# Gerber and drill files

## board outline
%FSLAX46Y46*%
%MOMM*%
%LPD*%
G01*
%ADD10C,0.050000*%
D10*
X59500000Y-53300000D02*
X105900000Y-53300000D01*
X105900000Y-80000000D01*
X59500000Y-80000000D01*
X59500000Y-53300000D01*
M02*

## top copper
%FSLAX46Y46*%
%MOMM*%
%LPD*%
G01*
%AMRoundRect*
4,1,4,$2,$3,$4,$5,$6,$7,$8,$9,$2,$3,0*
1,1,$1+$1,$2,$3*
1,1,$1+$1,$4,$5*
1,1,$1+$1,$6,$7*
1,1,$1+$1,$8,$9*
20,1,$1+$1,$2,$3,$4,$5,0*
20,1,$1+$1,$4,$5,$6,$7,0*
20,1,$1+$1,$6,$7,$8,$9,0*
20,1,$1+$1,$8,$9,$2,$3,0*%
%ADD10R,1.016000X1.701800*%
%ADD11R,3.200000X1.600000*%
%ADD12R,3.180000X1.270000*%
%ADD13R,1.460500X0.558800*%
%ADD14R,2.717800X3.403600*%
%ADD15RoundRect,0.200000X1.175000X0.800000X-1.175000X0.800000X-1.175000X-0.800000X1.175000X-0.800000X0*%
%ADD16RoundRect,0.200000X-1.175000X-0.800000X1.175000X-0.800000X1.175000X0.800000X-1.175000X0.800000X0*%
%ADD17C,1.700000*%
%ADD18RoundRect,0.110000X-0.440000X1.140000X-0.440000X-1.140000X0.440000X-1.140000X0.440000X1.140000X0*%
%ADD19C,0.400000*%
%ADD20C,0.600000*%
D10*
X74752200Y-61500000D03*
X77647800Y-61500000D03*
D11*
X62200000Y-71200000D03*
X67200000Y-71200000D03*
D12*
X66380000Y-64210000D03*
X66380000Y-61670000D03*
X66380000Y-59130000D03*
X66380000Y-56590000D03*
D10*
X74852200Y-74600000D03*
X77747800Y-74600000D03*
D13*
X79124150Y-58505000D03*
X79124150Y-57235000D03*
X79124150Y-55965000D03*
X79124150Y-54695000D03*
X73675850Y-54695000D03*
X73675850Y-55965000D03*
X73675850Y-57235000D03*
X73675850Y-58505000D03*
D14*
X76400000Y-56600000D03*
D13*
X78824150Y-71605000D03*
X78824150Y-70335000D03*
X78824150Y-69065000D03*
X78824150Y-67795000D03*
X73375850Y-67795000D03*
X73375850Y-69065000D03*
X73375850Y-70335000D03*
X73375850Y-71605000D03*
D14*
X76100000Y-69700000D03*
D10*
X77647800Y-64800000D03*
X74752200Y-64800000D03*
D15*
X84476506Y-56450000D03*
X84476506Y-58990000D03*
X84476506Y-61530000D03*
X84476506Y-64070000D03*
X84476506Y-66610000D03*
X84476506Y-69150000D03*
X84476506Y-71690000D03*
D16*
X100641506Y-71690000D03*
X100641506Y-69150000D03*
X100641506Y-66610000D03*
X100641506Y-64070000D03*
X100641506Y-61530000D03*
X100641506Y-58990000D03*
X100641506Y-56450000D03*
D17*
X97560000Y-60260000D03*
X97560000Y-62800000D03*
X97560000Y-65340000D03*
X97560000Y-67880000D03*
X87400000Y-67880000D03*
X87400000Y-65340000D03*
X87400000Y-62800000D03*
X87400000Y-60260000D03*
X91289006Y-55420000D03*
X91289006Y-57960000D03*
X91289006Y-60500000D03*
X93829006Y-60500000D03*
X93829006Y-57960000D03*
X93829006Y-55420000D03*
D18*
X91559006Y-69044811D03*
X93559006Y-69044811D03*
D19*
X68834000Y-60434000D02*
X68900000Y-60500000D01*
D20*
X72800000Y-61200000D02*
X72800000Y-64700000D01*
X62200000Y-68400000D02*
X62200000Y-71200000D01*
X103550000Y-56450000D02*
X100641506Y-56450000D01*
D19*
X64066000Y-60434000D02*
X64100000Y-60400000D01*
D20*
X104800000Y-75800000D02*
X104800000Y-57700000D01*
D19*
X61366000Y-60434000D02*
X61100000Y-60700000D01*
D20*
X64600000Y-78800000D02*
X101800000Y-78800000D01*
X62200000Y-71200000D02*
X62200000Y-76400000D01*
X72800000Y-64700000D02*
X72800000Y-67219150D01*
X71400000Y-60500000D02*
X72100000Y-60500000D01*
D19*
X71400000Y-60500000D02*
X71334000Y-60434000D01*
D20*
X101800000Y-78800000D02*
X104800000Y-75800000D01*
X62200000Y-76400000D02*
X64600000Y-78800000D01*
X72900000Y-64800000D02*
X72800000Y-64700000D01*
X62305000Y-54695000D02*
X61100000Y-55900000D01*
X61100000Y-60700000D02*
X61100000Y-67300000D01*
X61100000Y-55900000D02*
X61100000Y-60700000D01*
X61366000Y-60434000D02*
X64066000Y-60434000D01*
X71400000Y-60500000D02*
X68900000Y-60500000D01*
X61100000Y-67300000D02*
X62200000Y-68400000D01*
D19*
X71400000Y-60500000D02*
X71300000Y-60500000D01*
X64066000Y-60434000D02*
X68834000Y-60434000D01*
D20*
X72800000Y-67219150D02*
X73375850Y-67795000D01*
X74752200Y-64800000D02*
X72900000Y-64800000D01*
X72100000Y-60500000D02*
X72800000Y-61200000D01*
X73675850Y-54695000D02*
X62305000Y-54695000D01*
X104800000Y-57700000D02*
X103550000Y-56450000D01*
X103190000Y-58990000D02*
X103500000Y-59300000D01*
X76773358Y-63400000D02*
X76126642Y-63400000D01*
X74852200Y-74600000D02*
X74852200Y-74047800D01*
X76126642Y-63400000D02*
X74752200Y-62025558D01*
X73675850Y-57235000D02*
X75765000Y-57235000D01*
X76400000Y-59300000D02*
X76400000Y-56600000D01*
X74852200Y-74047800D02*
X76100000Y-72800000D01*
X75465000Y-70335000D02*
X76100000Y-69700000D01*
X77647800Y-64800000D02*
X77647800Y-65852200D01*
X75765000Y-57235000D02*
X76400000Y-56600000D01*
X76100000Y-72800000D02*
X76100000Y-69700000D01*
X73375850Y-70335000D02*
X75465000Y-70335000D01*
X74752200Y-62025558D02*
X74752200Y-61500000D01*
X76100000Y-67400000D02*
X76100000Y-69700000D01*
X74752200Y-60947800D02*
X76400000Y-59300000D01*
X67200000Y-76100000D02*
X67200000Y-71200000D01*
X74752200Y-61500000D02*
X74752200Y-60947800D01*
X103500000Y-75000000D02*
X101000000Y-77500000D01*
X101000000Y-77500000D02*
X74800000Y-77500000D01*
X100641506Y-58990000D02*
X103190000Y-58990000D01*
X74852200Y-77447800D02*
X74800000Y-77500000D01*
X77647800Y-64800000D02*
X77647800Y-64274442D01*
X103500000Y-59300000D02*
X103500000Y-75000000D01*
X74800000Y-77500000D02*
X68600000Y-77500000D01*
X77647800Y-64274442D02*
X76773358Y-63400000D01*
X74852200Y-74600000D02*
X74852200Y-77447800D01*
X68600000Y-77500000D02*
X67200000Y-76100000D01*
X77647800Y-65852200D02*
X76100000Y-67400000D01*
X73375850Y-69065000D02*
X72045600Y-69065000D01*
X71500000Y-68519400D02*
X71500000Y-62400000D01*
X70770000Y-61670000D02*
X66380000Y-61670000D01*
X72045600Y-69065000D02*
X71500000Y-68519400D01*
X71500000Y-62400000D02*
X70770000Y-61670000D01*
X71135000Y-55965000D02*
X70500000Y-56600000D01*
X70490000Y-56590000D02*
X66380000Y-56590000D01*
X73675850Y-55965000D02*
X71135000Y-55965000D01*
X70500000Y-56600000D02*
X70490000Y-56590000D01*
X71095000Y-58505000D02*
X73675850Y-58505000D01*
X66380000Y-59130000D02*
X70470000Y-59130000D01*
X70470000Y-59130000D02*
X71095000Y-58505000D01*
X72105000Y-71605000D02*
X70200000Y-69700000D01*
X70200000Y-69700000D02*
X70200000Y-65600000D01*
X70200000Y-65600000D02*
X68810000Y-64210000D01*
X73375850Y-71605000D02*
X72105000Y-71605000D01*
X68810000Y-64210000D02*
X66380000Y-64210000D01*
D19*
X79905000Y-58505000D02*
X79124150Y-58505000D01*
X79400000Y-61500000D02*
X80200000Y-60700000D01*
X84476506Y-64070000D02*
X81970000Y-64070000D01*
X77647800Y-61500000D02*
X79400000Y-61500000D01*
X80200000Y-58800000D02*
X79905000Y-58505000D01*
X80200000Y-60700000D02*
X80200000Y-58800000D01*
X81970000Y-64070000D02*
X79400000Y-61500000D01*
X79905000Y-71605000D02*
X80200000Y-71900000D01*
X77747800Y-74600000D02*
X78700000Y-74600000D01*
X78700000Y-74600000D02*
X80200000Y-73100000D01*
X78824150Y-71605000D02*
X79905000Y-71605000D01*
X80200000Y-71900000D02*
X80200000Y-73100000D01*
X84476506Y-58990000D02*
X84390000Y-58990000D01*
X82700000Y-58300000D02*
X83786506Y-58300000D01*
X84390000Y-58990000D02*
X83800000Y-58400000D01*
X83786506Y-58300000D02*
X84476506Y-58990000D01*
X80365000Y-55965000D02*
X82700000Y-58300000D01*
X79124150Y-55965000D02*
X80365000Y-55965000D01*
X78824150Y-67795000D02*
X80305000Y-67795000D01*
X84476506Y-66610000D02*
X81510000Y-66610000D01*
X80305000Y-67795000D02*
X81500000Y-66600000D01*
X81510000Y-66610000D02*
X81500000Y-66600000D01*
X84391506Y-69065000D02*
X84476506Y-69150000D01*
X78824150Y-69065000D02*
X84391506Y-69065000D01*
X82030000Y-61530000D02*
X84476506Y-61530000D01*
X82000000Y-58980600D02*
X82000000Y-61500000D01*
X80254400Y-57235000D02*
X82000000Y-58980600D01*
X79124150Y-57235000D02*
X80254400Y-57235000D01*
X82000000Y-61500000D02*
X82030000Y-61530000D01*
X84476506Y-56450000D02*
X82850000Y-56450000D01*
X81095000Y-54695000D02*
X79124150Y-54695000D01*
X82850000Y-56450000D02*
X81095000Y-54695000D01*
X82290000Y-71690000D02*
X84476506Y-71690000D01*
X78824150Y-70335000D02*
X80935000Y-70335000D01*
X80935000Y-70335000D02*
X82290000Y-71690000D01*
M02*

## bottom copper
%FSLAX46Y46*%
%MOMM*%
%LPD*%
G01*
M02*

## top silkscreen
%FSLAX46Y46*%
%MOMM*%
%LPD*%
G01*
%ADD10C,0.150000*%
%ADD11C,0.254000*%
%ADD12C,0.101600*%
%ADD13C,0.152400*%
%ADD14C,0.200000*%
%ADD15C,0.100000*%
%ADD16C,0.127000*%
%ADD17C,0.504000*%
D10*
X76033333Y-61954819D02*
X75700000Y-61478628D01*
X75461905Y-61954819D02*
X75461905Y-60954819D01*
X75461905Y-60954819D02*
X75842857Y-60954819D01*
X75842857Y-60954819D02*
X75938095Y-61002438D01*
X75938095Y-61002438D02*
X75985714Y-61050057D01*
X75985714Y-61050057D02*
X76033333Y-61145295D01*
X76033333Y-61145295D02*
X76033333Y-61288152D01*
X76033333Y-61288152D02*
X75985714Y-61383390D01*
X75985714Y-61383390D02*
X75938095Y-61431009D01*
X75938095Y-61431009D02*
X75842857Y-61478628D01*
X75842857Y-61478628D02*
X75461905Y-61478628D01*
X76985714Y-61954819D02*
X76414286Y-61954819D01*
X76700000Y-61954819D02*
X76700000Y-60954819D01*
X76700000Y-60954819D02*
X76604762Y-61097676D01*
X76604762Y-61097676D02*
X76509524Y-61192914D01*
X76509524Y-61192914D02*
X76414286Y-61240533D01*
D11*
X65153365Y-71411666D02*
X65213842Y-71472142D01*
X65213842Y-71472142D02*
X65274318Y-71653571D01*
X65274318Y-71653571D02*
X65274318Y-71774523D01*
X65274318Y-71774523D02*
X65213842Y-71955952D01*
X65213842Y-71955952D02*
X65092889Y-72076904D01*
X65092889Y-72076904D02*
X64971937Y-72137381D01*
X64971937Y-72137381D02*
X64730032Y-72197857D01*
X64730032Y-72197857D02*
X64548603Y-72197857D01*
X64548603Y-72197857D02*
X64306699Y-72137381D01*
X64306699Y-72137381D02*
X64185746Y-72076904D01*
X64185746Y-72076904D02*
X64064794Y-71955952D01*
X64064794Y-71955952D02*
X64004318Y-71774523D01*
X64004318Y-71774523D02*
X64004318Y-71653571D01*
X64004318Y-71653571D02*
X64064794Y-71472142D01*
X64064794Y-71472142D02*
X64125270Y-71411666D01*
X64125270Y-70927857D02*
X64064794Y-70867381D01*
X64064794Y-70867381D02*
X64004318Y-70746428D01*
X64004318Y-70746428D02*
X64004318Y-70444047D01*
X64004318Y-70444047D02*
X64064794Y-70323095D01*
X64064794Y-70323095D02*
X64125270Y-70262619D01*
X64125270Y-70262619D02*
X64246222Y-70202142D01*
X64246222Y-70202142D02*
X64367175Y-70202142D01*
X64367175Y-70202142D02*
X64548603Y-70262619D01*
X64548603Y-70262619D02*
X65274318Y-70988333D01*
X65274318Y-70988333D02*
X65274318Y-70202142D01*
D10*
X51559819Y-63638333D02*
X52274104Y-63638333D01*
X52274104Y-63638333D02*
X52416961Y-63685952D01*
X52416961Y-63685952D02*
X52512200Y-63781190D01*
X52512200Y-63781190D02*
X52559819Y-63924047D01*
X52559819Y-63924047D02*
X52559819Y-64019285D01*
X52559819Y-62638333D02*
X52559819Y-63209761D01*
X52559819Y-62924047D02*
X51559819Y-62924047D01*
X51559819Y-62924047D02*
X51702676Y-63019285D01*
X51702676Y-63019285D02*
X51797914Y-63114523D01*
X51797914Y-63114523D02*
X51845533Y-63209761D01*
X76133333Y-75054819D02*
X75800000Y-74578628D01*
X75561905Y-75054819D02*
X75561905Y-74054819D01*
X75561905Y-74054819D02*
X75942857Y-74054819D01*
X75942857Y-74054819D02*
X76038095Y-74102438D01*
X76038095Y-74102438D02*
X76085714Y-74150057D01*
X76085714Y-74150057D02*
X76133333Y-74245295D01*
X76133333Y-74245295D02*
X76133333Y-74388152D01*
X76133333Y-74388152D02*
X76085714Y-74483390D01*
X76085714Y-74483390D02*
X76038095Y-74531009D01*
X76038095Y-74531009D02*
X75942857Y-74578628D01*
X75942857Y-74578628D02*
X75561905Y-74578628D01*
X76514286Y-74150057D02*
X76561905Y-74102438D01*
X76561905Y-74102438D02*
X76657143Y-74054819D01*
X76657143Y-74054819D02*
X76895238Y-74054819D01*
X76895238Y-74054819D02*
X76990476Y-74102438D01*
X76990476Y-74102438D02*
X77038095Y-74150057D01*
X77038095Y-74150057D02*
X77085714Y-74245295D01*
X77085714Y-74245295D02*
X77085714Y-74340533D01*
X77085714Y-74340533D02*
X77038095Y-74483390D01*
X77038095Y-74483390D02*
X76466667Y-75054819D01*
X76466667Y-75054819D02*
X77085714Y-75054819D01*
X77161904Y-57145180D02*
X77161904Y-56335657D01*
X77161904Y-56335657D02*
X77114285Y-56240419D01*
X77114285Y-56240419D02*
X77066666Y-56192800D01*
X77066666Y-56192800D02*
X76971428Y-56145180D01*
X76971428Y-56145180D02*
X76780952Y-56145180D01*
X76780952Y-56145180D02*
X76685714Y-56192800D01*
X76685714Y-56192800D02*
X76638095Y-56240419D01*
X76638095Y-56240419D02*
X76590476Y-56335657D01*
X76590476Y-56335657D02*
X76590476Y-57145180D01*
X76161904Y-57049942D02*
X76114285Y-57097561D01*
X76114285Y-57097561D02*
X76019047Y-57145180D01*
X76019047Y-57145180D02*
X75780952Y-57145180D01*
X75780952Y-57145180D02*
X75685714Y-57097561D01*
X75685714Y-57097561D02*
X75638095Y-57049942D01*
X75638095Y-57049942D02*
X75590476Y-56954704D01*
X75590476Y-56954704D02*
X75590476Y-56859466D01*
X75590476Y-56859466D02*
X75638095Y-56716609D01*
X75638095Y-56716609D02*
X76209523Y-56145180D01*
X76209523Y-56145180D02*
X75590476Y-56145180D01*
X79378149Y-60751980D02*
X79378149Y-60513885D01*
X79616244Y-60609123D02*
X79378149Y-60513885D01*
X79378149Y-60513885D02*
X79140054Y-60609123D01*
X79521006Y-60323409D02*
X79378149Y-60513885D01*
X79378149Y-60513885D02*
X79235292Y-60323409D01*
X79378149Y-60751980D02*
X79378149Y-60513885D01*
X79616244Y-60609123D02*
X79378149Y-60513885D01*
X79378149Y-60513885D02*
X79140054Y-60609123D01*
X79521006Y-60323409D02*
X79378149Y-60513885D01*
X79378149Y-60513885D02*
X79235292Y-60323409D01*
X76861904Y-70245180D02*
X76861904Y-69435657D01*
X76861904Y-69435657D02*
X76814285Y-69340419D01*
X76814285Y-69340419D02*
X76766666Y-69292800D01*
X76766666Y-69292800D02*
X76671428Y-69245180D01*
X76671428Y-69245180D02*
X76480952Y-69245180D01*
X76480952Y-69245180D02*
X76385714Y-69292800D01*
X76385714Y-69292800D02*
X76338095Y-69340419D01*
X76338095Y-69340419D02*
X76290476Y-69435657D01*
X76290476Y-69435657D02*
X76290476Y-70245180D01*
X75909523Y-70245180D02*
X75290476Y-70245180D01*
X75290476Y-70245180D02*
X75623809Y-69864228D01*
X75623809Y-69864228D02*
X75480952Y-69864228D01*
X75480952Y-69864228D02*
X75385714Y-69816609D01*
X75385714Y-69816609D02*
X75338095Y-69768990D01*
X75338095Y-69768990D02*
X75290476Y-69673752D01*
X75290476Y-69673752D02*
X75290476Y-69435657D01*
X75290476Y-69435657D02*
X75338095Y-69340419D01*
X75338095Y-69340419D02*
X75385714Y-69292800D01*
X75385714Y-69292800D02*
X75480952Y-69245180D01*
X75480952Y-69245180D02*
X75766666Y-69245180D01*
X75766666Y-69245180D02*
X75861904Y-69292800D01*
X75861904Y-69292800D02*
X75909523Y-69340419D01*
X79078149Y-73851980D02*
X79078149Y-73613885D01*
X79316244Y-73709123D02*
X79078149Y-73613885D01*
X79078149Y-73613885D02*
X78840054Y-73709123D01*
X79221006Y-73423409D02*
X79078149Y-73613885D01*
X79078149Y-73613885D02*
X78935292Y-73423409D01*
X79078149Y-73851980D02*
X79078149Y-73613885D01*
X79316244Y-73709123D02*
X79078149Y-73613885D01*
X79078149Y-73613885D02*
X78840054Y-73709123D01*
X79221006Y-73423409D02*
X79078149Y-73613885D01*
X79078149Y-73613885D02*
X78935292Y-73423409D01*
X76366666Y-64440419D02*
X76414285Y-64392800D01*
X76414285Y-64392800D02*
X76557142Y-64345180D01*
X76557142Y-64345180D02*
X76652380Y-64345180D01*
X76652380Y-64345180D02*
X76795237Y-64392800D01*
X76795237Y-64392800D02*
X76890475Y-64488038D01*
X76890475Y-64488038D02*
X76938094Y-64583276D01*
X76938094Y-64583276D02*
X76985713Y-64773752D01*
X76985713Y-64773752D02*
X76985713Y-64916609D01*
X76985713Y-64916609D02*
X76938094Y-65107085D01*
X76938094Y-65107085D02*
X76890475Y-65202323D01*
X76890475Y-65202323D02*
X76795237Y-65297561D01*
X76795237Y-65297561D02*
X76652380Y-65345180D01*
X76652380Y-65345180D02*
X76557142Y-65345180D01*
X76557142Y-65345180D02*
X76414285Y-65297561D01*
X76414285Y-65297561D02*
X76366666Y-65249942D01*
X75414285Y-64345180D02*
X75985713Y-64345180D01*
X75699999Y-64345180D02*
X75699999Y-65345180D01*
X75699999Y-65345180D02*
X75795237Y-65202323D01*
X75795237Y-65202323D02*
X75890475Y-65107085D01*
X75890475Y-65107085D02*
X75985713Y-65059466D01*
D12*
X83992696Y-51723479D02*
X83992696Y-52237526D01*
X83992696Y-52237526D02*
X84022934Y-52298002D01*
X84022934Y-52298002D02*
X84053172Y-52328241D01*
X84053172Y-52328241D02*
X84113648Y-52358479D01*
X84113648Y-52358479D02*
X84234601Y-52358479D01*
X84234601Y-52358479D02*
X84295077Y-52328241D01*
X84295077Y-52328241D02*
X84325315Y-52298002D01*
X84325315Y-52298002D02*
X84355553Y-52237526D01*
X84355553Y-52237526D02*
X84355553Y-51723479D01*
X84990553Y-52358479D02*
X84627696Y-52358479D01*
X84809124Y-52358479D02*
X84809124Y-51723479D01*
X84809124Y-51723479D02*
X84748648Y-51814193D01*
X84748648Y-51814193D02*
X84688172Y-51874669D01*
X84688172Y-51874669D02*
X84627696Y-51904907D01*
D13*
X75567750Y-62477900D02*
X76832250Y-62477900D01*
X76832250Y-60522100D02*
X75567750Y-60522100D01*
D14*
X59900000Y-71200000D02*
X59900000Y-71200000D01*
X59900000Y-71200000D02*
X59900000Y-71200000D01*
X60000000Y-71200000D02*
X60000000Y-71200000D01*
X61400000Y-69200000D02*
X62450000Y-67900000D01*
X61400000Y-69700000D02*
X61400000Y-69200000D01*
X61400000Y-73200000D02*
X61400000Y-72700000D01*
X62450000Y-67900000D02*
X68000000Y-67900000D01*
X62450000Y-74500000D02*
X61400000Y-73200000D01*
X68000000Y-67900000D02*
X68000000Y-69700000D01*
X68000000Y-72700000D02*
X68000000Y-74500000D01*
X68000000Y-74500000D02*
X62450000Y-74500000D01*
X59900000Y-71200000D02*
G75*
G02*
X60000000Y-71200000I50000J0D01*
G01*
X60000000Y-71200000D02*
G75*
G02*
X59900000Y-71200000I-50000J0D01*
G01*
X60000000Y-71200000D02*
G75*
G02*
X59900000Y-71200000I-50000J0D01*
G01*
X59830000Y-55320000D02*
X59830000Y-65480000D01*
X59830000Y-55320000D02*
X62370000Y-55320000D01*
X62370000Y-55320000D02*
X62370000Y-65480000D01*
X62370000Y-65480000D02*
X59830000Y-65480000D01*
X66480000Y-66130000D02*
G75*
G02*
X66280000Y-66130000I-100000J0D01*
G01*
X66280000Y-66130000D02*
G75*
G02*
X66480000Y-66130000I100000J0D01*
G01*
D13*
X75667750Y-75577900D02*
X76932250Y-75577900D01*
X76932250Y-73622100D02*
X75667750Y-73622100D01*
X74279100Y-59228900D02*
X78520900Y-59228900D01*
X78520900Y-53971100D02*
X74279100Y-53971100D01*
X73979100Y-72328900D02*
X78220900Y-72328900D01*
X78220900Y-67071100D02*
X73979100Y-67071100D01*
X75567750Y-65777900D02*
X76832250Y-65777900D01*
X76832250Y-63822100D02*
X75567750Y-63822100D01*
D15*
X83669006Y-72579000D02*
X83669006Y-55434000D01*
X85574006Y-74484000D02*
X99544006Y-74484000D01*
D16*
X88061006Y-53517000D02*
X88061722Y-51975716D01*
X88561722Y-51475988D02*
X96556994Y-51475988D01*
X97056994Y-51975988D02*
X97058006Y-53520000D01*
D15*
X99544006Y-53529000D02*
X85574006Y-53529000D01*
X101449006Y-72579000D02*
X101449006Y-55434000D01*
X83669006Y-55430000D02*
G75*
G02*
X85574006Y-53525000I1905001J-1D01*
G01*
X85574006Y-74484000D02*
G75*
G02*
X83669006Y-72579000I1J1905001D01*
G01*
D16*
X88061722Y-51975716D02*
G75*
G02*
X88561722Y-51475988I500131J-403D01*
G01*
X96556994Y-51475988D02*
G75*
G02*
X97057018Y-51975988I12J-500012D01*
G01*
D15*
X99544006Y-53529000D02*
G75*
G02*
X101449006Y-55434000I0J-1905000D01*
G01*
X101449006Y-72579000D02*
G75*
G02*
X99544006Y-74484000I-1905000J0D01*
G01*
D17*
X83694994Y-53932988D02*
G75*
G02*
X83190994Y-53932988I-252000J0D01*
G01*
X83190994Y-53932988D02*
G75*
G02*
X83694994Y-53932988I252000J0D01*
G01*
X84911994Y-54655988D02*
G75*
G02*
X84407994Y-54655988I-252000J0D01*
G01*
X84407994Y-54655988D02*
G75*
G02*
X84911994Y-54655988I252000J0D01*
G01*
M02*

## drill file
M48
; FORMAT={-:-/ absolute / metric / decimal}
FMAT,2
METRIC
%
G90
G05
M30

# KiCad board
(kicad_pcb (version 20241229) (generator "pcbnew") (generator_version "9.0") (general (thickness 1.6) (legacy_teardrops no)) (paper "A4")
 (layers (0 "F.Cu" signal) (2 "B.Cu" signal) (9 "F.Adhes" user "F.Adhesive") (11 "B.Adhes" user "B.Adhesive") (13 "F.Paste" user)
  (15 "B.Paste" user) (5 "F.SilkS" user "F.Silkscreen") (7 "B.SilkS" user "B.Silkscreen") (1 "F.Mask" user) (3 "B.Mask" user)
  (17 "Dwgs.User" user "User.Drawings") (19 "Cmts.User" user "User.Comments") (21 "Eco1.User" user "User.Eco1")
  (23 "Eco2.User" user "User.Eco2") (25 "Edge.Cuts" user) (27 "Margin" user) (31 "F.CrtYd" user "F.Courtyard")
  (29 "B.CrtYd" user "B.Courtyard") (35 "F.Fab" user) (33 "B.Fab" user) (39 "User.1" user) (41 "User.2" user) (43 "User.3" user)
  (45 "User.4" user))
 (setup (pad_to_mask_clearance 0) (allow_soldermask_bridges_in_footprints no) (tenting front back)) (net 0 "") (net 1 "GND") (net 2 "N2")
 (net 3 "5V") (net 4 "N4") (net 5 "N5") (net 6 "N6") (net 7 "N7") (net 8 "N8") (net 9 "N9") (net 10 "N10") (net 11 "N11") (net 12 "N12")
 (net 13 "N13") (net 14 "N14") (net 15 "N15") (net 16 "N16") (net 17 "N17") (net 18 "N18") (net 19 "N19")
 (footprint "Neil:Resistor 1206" (layer "F.Cu") (at 76.2 61.5)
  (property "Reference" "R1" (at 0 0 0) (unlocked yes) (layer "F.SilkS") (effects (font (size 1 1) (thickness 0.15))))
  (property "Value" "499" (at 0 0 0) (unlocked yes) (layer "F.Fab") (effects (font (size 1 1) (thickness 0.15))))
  (fp_line (start -0.63225 0.9779) (end 0.63225 0.9779) (stroke (width 0.1524) (type solid)) (layer "F.SilkS"))
  (fp_line (start 0.63225 -0.9779) (end -0.63225 -0.9779) (stroke (width 0.1524) (type solid)) (layer "F.SilkS"))
  (pad "1" smd rect (at -1.4478 0) (size 1.016 1.7018) (layers "F.Cu" "F.Mask" "F.Paste") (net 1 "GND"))
  (pad "2" smd rect (at 1.4478 0) (size 1.016 1.7018) (layers "F.Cu" "F.Mask" "F.Paste") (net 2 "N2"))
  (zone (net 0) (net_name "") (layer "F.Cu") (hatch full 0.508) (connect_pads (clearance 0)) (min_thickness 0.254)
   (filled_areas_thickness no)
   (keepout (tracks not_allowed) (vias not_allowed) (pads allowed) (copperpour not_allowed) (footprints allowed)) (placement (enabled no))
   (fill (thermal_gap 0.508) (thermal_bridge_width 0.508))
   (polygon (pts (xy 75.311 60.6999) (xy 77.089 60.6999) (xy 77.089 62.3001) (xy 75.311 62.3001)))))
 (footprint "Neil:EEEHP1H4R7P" (layer "F.Cu") (at 64.7 71.2 -90)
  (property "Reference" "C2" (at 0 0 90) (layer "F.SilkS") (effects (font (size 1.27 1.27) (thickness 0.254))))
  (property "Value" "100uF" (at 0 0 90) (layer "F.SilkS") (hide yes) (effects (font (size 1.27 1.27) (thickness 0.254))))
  (fp_line (start 0 4.8) (end 0 4.8) (stroke (width 0.2) (type solid)) (layer "F.SilkS"))
  (fp_line (start 0 4.8) (end 0 4.8) (stroke (width 0.2) (type solid)) (layer "F.SilkS"))
  (fp_line (start 0 4.7) (end 0 4.7) (stroke (width 0.2) (type solid)) (layer "F.SilkS"))
  (fp_line (start -2 3.3) (end -3.3 2.25) (stroke (width 0.2) (type solid)) (layer "F.SilkS"))
  (fp_line (start -1.5 3.3) (end -2 3.3) (stroke (width 0.2) (type solid)) (layer "F.SilkS"))
  (fp_line (start 2 3.3) (end 1.5 3.3) (stroke (width 0.2) (type solid)) (layer "F.SilkS"))
  (fp_line (start -3.3 2.25) (end -3.3 -3.3) (stroke (width 0.2) (type solid)) (layer "F.SilkS"))
  (fp_line (start 3.3 2.25) (end 2 3.3) (stroke (width 0.2) (type solid)) (layer "F.SilkS"))
  (fp_line (start -3.3 -3.3) (end -1.5 -3.3) (stroke (width 0.2) (type solid)) (layer "F.SilkS"))
  (fp_line (start 1.5 -3.3) (end 3.3 -3.3) (stroke (width 0.2) (type solid)) (layer "F.SilkS"))
  (fp_line (start 3.3 -3.3) (end 3.3 2.25) (stroke (width 0.2) (type solid)) (layer "F.SilkS"))
  (fp_arc (start 0 4.8) (mid -0.05 4.75) (end 0 4.7) (stroke (width 0.2) (type solid)) (layer "F.SilkS"))
  (fp_arc (start 0 4.7) (mid 0.05 4.75) (end 0 4.8) (stroke (width 0.2) (type solid)) (layer "F.SilkS"))
  (fp_arc (start 0 4.7) (mid 0.05 4.75) (end 0 4.8) (stroke (width 0.2) (type solid)) (layer "F.SilkS"))
  (pad "1" smd rect (at 0 2.5 270) (size 1.6 3.2) (layers "F.Cu" "F.Mask" "F.Paste") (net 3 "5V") (thermal_bridge_angle 45))
  (pad "2" smd rect (at 0 -2.5 270) (size 1.6 3.2) (layers "F.Cu" "F.Mask" "F.Paste") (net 1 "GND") (thermal_bridge_angle 45)))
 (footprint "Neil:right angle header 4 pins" (layer "F.Cu") (at 61.1 60.4 90)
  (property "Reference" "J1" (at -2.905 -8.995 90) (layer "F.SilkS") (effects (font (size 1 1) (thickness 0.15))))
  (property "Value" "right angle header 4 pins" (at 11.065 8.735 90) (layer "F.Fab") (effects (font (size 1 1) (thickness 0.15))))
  (fp_line (start 5.08 -1.27) (end -5.08 -1.27) (stroke (width 0.2) (type solid)) (layer "F.SilkS"))
  (fp_line (start 5.08 -1.27) (end 5.08 1.27) (stroke (width 0.2) (type solid)) (layer "F.SilkS"))
  (fp_line (start 5.08 1.27) (end -5.08 1.27) (stroke (width 0.2) (type solid)) (layer "F.SilkS"))
  (fp_line (start -5.08 1.27) (end -5.08 -1.27) (stroke (width 0.2) (type solid)) (layer "F.SilkS"))
  (fp_circle (center -5.73 5.28) (end -5.63 5.28) (stroke (width 0.2) (type solid)) (fill no) (layer "F.SilkS"))
  (pad "01" smd rect (at -3.81 5.28 90) (size 1.27 3.18) (layers "F.Cu" "F.Mask" "F.Paste") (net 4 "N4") (solder_mask_margin 0.102))
  (pad "02" smd rect (at -1.27 5.28 90) (size 1.27 3.18) (layers "F.Cu" "F.Mask" "F.Paste") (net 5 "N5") (solder_mask_margin 0.102))
  (pad "03" smd rect (at 1.27 5.28 90) (size 1.27 3.18) (layers "F.Cu" "F.Mask" "F.Paste") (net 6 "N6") (solder_mask_margin 0.102))
  (pad "04" smd rect (at 3.81 5.28 90) (size 1.27 3.18) (layers "F.Cu" "F.Mask" "F.Paste") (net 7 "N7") (solder_mask_margin 0.102)))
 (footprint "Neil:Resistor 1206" (layer "F.Cu") (at 76.3 74.6)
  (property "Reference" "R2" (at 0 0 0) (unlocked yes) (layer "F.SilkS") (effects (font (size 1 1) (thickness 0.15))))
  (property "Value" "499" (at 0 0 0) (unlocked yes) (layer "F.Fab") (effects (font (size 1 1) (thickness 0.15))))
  (fp_line (start -0.63225 0.9779) (end 0.63225 0.9779) (stroke (width 0.1524) (type solid)) (layer "F.SilkS"))
  (fp_line (start 0.63225 -0.9779) (end -0.63225 -0.9779) (stroke (width 0.1524) (type solid)) (layer "F.SilkS"))
  (pad "1" smd rect (at -1.4478 0) (size 1.016 1.7018) (layers "F.Cu" "F.Mask" "F.Paste") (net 1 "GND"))
  (pad "2" smd rect (at 1.4478 0) (size 1.016 1.7018) (layers "F.Cu" "F.Mask" "F.Paste") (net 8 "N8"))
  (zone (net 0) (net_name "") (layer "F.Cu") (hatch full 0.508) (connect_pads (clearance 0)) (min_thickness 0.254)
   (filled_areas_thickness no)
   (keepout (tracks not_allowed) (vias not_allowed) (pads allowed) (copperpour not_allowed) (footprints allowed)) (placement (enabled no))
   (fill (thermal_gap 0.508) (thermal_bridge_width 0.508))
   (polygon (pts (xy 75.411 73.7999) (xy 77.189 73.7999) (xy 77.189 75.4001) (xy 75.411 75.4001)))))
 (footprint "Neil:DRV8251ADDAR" (layer "F.Cu") (at 76.4 56.6 180)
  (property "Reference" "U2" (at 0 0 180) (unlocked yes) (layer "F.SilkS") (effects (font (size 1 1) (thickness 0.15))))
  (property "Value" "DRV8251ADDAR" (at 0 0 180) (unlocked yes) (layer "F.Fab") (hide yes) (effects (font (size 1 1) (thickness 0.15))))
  (fp_line (start 2.1209 -2.6289) (end -2.1209 -2.6289) (stroke (width 0.1524) (type solid)) (layer "F.SilkS"))
  (fp_line (start -2.1209 2.6289) (end 2.1209 2.6289) (stroke (width 0.1524) (type solid)) (layer "F.SilkS"))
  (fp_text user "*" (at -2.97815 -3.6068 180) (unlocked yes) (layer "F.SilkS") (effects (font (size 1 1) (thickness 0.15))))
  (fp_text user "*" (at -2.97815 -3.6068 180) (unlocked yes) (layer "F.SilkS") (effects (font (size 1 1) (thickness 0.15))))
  (pad "1" smd rect (at -2.72415 -1.905 180) (size 1.4605 0.5588) (layers "F.Cu" "F.Mask" "F.Paste") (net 2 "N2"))
  (pad "2" smd rect (at -2.72415 -0.635 180) (size 1.4605 0.5588) (layers "F.Cu" "F.Mask" "F.Paste") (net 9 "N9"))
  (pad "3" smd rect (at -2.72415 0.635 180) (size 1.4605 0.5588) (layers "F.Cu" "F.Mask" "F.Paste") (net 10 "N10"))
  (pad "4" smd rect (at -2.72415 1.905 180) (size 1.4605 0.5588) (layers "F.Cu" "F.Mask" "F.Paste") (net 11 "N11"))
  (pad "5" smd rect (at 2.72415 1.905 180) (size 1.4605 0.5588) (layers "F.Cu" "F.Mask" "F.Paste") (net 3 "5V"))
  (pad "6" smd rect (at 2.72415 0.635 180) (size 1.4605 0.5588) (layers "F.Cu" "F.Mask" "F.Paste") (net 7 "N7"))
  (pad "7" smd rect (at 2.72415 -0.635 180) (size 1.4605 0.5588) (layers "F.Cu" "F.Mask" "F.Paste") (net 1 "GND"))
  (pad "8" smd rect (at 2.72415 -1.905 180) (size 1.4605 0.5588) (layers "F.Cu" "F.Mask" "F.Paste") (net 6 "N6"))
  (pad "9" smd rect (at 0 0 180) (size 2.7178 3.4036) (layers "F.Cu" "F.Mask") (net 1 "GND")))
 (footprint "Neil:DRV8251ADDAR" (layer "F.Cu") (at 76.1 69.7 180)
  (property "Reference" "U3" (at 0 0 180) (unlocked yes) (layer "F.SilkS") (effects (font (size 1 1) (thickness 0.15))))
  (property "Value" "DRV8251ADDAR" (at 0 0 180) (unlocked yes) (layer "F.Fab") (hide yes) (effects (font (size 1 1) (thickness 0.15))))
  (fp_line (start 2.1209 -2.6289) (end -2.1209 -2.6289) (stroke (width 0.1524) (type solid)) (layer "F.SilkS"))
  (fp_line (start -2.1209 2.6289) (end 2.1209 2.6289) (stroke (width 0.1524) (type solid)) (layer "F.SilkS"))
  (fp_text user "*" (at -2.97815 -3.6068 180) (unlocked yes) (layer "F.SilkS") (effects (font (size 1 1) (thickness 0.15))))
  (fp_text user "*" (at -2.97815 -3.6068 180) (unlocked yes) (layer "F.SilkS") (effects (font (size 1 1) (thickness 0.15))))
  (pad "1" smd rect (at -2.72415 -1.905 180) (size 1.4605 0.5588) (layers "F.Cu" "F.Mask" "F.Paste") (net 8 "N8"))
  (pad "2" smd rect (at -2.72415 -0.635 180) (size 1.4605 0.5588) (layers "F.Cu" "F.Mask" "F.Paste") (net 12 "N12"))
  (pad "3" smd rect (at -2.72415 0.635 180) (size 1.4605 0.5588) (layers "F.Cu" "F.Mask" "F.Paste") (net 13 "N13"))
  (pad "4" smd rect (at -2.72415 1.905 180) (size 1.4605 0.5588) (layers "F.Cu" "F.Mask" "F.Paste") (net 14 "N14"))
  (pad "5" smd rect (at 2.72415 1.905 180) (size 1.4605 0.5588) (layers "F.Cu" "F.Mask" "F.Paste") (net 3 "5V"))
  (pad "6" smd rect (at 2.72415 0.635 180) (size 1.4605 0.5588) (layers "F.Cu" "F.Mask" "F.Paste") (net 5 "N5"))
  (pad "7" smd rect (at 2.72415 -0.635 180) (size 1.4605 0.5588) (layers "F.Cu" "F.Mask" "F.Paste") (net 1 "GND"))
  (pad "8" smd rect (at 2.72415 -1.905 180) (size 1.4605 0.5588) (layers "F.Cu" "F.Mask" "F.Paste") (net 4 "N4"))
  (pad "9" smd rect (at 0 0 180) (size 2.7178 3.4036) (layers "F.Cu" "F.Mask") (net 1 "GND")))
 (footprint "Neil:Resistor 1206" (layer "F.Cu") (at 76.2 64.8 180)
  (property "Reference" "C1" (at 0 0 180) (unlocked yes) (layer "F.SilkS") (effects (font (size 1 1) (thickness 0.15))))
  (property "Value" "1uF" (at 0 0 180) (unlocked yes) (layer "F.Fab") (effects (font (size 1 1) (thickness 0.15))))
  (fp_line (start 0.63225 -0.9779) (end -0.63225 -0.9779) (stroke (width 0.1524) (type solid)) (layer "F.SilkS"))
  (fp_line (start -0.63225 0.9779) (end 0.63225 0.9779) (stroke (width 0.1524) (type solid)) (layer "F.SilkS"))
  (pad "1" smd rect (at -1.4478 0 180) (size 1.016 1.7018) (layers "F.Cu" "F.Mask" "F.Paste") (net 1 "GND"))
  (pad "2" smd rect (at 1.4478 0 180) (size 1.016 1.7018) (layers "F.Cu" "F.Mask" "F.Paste") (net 3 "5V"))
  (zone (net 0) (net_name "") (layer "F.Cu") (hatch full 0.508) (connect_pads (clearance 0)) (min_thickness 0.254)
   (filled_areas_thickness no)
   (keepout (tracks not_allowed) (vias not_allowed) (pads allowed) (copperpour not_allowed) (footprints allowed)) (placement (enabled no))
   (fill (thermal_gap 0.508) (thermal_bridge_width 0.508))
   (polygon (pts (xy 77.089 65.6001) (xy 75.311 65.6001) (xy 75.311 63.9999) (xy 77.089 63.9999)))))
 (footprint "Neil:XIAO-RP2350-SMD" (layer "F.Cu") (at 92.476506 64.07)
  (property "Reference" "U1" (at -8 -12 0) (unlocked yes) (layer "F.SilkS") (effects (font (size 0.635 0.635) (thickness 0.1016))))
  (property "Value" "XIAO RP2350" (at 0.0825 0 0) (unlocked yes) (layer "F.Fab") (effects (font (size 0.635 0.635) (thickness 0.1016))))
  (fp_line (start -8.8075 8.509) (end -8.8075 -8.636) (stroke (width 0.1) (type solid)) (layer "F.SilkS"))
  (fp_line (start -6.9025 10.414) (end 7.0675 10.414) (stroke (width 0.1) (type solid)) (layer "F.SilkS"))
  (fp_line (start -4.4155 -10.553) (end -4.414784 -12.094284) (stroke (width 0.127) (type solid)) (layer "F.SilkS"))
  (fp_line (start -3.914784 -12.594012) (end 4.080488 -12.594012) (stroke (width 0.127) (type solid)) (layer "F.SilkS"))
  (fp_line (start 4.580488 -12.094012) (end 4.5815 -10.55) (stroke (width 0.127) (type solid)) (layer "F.SilkS"))
  (fp_line (start 7.0675 -10.541) (end -6.9025 -10.541) (stroke (width 0.1) (type solid)) (layer "F.SilkS"))
  (fp_line (start 8.9725 8.509) (end 8.9725 -8.636) (stroke (width 0.1) (type solid)) (layer "F.SilkS"))
  (fp_arc (start -8.8075 -8.64) (mid -8.249538 -9.987038) (end -6.9025 -10.545) (stroke (width 0.1) (type solid)) (layer "F.SilkS"))
  (fp_arc (start -6.9025 10.414) (mid -8.249538 9.856038) (end -8.8075 8.509) (stroke (width 0.1) (type solid)) (layer "F.SilkS"))
  (fp_arc (start -4.414784 -12.094284) (mid -4.268207 -12.447619) (end -3.914784 -12.594012) (stroke (width 0.127) (type default))
   (layer "F.SilkS"))
  (fp_arc (start 4.080488 -12.594012) (mid 4.434053 -12.44757) (end 4.580488 -12.094012) (stroke (width 0.127) (type default))
   (layer "F.SilkS"))
  (fp_arc (start 7.0675 -10.541) (mid 8.414538 -9.983038) (end 8.9725 -8.636) (stroke (width 0.1) (type solid)) (layer "F.SilkS"))
  (fp_arc (start 8.9725 8.509) (mid 8.414538 9.856038) (end 7.0675 10.414) (stroke (width 0.1) (type solid)) (layer "F.SilkS"))
  (fp_circle (center -9.033512 -10.137012) (end -9.033512 -10.391012) (stroke (width 0.5) (type solid)) (fill yes) (layer "F.SilkS"))
  (fp_circle (center -7.816512 -9.414012) (end -7.816512 -9.668012) (stroke (width 0.5) (type solid)) (fill yes) (layer "F.SilkS"))
  (pad "1" smd roundrect (at -8 -7.62 180) (size 2.75 2) (layers "F.Cu" "F.Mask" "F.Paste") (roundrect_rratio 0.1) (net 11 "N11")
   (thermal_bridge_angle 45))
  (pad "2" smd roundrect (at -8 -5.08 180) (size 2.75 2) (layers "F.Cu" "F.Mask" "F.Paste") (roundrect_rratio 0.1) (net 10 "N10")
   (thermal_bridge_angle 45))
  (pad "3" smd roundrect (at -8 -2.54 180) (size 2.75 2) (layers "F.Cu" "F.Mask" "F.Paste") (roundrect_rratio 0.1) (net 9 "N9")
   (thermal_bridge_angle 45))
  (pad "4" smd roundrect (at -8 0 180) (size 2.75 2) (layers "F.Cu" "F.Mask" "F.Paste") (roundrect_rratio 0.1) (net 2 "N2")
   (thermal_bridge_angle 45))
  (pad "5" smd roundrect (at -8 2.54 180) (size 2.75 2) (layers "F.Cu" "F.Mask" "F.Paste") (roundrect_rratio 0.1) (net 14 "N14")
   (thermal_bridge_angle 45))
  (pad "6" smd roundrect (at -8 5.08 180) (size 2.75 2) (layers "F.Cu" "F.Mask" "F.Paste") (roundrect_rratio 0.1) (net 13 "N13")
   (thermal_bridge_angle 45))
  (pad "7" smd roundrect (at -8 7.62 180) (size 2.75 2) (layers "F.Cu" "F.Mask" "F.Paste") (roundrect_rratio 0.1) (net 12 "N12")
   (thermal_bridge_angle 45))
  (pad "8" smd roundrect (at 8.165 7.62) (size 2.75 2) (layers "F.Cu" "F.Mask" "F.Paste") (roundrect_rratio 0.1) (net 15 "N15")
   (thermal_bridge_angle 45))
  (pad "9" smd roundrect (at 8.165 5.08) (size 2.75 2) (layers "F.Cu" "F.Mask" "F.Paste") (roundrect_rratio 0.1) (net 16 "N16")
   (thermal_bridge_angle 45))
  (pad "10" smd roundrect (at 8.165 2.54) (size 2.75 2) (layers "F.Cu" "F.Mask" "F.Paste") (roundrect_rratio 0.1) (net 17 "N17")
   (thermal_bridge_angle 45))
  (pad "11" smd roundrect (at 8.165 0) (size 2.75 2) (layers "F.Cu" "F.Mask" "F.Paste") (roundrect_rratio 0.1) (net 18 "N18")
   (thermal_bridge_angle 45))
  (pad "12" smd roundrect (at 8.165 -2.54) (size 2.75 2) (layers "F.Cu" "F.Mask" "F.Paste") (roundrect_rratio 0.1) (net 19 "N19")
   (thermal_bridge_angle 45))
  (pad "13" smd roundrect (at 8.165 -5.08) (size 2.75 2) (layers "F.Cu" "F.Mask" "F.Paste") (roundrect_rratio 0.1) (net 1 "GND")
   (thermal_bridge_angle 45))
  (pad "14" smd roundrect (at 8.165 -7.62) (size 2.75 2) (layers "F.Cu" "F.Mask" "F.Paste") (roundrect_rratio 0.1) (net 3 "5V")
   (thermal_bridge_angle 45))
  (pad "15" smd circle (at 5.083494 -3.81 180) (size 1.7 1.7) (layers "F.Cu" "F.Mask" "F.Paste"))
  (pad "16" smd circle (at 5.083494 -1.27 180) (size 1.7 1.7) (layers "F.Cu" "F.Mask" "F.Paste"))
  (pad "17" smd circle (at 5.083494 1.27 180) (size 1.7 1.7) (layers "F.Cu" "F.Mask" "F.Paste"))
  (pad "18" smd circle (at 5.083494 3.81 180) (size 1.7 1.7) (layers "F.Cu" "F.Mask" "F.Paste"))
  (pad "19" smd circle (at -5.076506 3.81 180) (size 1.7 1.7) (layers "F.Cu" "F.Mask" "F.Paste"))
  (pad "20" smd circle (at -5.076506 1.27 180) (size 1.7 1.7) (layers "F.Cu" "F.Mask" "F.Paste"))
  (pad "21" smd circle (at -5.076506 -1.27 180) (size 1.7 1.7) (layers "F.Cu" "F.Mask" "F.Paste"))
  (pad "22" smd circle (at -5.076506 -3.81 180) (size 1.7 1.7) (layers "F.Cu" "F.Mask" "F.Paste"))
  (pad "23" smd circle (at -1.1875 -8.65 180) (size 1.7 1.7) (layers "F.Cu" "F.Mask" "F.Paste"))
  (pad "24" smd circle (at -1.1875 -6.11 180) (size 1.7 1.7) (layers "F.Cu" "F.Mask" "F.Paste"))
  (pad "25" smd circle (at -1.1875 -3.57 180) (size 1.7 1.7) (layers "F.Cu" "F.Mask" "F.Paste"))
  (pad "26" smd circle (at 1.3525 -3.57 180) (size 1.7 1.7) (layers "F.Cu" "F.Mask" "F.Paste"))
  (pad "27" smd circle (at 1.3525 -6.11 180) (size 1.7 1.7) (layers "F.Cu" "F.Mask" "F.Paste"))
  (pad "28" smd circle (at 1.3525 -8.65 180) (size 1.7 1.7) (layers "F.Cu" "F.Mask" "F.Paste"))
  (pad "29" smd roundrect (at -0.9175 4.974811 270) (size 2.5 1.1) (layers "F.Cu" "F.Mask" "F.Paste") (roundrect_rratio 0.1)
   (thermal_bridge_angle 45))
  (pad "30" smd roundrect (at 1.0825 4.974811 270) (size 2.5 1.1) (layers "F.Cu" "F.Mask" "F.Paste") (roundrect_rratio 0.1)
   (thermal_bridge_angle 45)))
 (gr_rect (start 59.5 53.3) (end 105.9 80) (stroke (width 0.05) (type default)) (fill no) (layer "Edge.Cuts"))
 (segment (start 68.834 60.434) (end 68.9 60.5) (width 0.4) (layer "F.Cu") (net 3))
 (segment (start 72.8 61.2) (end 72.8 64.7) (width 0.6) (layer "F.Cu") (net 3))
 (segment (start 62.2 68.4) (end 62.2 71.2) (width 0.6) (layer "F.Cu") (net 3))
 (segment (start 103.55 56.45) (end 100.641506 56.45) (width 0.6) (layer "F.Cu") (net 3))
 (segment (start 64.066 60.434) (end 64.1 60.4) (width 0.4) (layer "F.Cu") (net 3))
 (segment (start 104.8 75.8) (end 104.8 57.7) (width 0.6) (layer "F.Cu") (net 3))
 (segment (start 61.366 60.434) (end 61.1 60.7) (width 0.4) (layer "F.Cu") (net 3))
 (segment (start 64.6 78.8) (end 101.8 78.8) (width 0.6) (layer "F.Cu") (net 3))
 (segment (start 62.2 71.2) (end 62.2 76.4) (width 0.6) (layer "F.Cu") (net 3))
 (segment (start 72.8 64.7) (end 72.8 67.21915) (width 0.6) (layer "F.Cu") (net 3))
 (segment (start 71.4 60.5) (end 72.1 60.5) (width 0.6) (layer "F.Cu") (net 3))
 (segment (start 71.4 60.5) (end 71.334 60.434) (width 0.4) (layer "F.Cu") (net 3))
 (segment (start 101.8 78.8) (end 104.8 75.8) (width 0.6) (layer "F.Cu") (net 3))
 (segment (start 62.2 76.4) (end 64.6 78.8) (width 0.6) (layer "F.Cu") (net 3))
 (segment (start 72.9 64.8) (end 72.8 64.7) (width 0.6) (layer "F.Cu") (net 3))
 (segment (start 62.305 54.695) (end 61.1 55.9) (width 0.6) (layer "F.Cu") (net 3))
 (segment (start 61.1 60.7) (end 61.1 67.3) (width 0.6) (layer "F.Cu") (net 3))
 (segment (start 61.1 55.9) (end 61.1 60.7) (width 0.6) (layer "F.Cu") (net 3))
 (segment (start 61.366 60.434) (end 64.066 60.434) (width 0.6) (layer "F.Cu") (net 3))
 (segment (start 71.4 60.5) (end 68.9 60.5) (width 0.6) (layer "F.Cu") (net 3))
 (segment (start 61.1 67.3) (end 62.2 68.4) (width 0.6) (layer "F.Cu") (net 3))
 (segment (start 71.4 60.5) (end 71.3 60.5) (width 0.4) (layer "F.Cu") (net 3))
 (segment (start 64.066 60.434) (end 68.834 60.434) (width 0.4) (layer "F.Cu") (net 3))
 (segment (start 72.8 67.21915) (end 73.37585 67.795) (width 0.6) (layer "F.Cu") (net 3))
 (segment (start 74.7522 64.8) (end 72.9 64.8) (width 0.6) (layer "F.Cu") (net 3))
 (segment (start 72.1 60.5) (end 72.8 61.2) (width 0.6) (layer "F.Cu") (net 3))
 (segment (start 73.67585 54.695) (end 62.305 54.695) (width 0.6) (layer "F.Cu") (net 3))
 (segment (start 104.8 57.7) (end 103.55 56.45) (width 0.6) (layer "F.Cu") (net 3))
 (segment (start 103.19 58.99) (end 103.5 59.3) (width 0.6) (layer "F.Cu") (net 1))
 (segment (start 76.773358 63.4) (end 76.126642 63.4) (width 0.6) (layer "F.Cu") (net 1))
 (segment (start 74.8522 74.6) (end 74.8522 74.0478) (width 0.6) (layer "F.Cu") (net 1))
 (segment (start 76.126642 63.4) (end 74.7522 62.025558) (width 0.6) (layer "F.Cu") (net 1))
 (segment (start 73.67585 57.235) (end 75.765 57.235) (width 0.6) (layer "F.Cu") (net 1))
 (segment (start 76.4 59.3) (end 76.4 56.6) (width 0.6) (layer "F.Cu") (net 1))
 (segment (start 74.8522 74.0478) (end 76.1 72.8) (width 0.6) (layer "F.Cu") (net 1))
 (segment (start 75.465 70.335) (end 76.1 69.7) (width 0.6) (layer "F.Cu") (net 1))
 (segment (start 77.6478 64.8) (end 77.6478 65.8522) (width 0.6) (layer "F.Cu") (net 1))
 (segment (start 75.765 57.235) (end 76.4 56.6) (width 0.6) (layer "F.Cu") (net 1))
 (segment (start 76.1 72.8) (end 76.1 69.7) (width 0.6) (layer "F.Cu") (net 1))
 (segment (start 73.37585 70.335) (end 75.465 70.335) (width 0.6) (layer "F.Cu") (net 1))
 (segment (start 74.7522 62.025558) (end 74.7522 61.5) (width 0.6) (layer "F.Cu") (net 1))
 (segment (start 76.1 67.4) (end 76.1 69.7) (width 0.6) (layer "F.Cu") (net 1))
 (segment (start 74.7522 60.9478) (end 76.4 59.3) (width 0.6) (layer "F.Cu") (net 1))
 (segment (start 67.2 76.1) (end 67.2 71.2) (width 0.6) (layer "F.Cu") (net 1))
 (segment (start 74.7522 61.5) (end 74.7522 60.9478) (width 0.6) (layer "F.Cu") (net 1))
 (segment (start 103.5 75) (end 101 77.5) (width 0.6) (layer "F.Cu") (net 1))
 (segment (start 101 77.5) (end 74.8 77.5) (width 0.6) (layer "F.Cu") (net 1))
 (segment (start 100.641506 58.99) (end 103.19 58.99) (width 0.6) (layer "F.Cu") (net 1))
 (segment (start 74.8522 77.4478) (end 74.8 77.5) (width 0.6) (layer "F.Cu") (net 1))
 (segment (start 77.6478 64.8) (end 77.6478 64.274442) (width 0.6) (layer "F.Cu") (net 1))
 (segment (start 103.5 59.3) (end 103.5 75) (width 0.6) (layer "F.Cu") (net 1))
 (segment (start 74.8 77.5) (end 68.6 77.5) (width 0.6) (layer "F.Cu") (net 1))
 (segment (start 77.6478 64.274442) (end 76.773358 63.4) (width 0.6) (layer "F.Cu") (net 1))
 (segment (start 74.8522 74.6) (end 74.8522 77.4478) (width 0.6) (layer "F.Cu") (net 1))
 (segment (start 68.6 77.5) (end 67.2 76.1) (width 0.6) (layer "F.Cu") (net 1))
 (segment (start 77.6478 65.8522) (end 76.1 67.4) (width 0.6) (layer "F.Cu") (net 1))
 (segment (start 73.37585 69.065) (end 72.0456 69.065) (width 0.6) (layer "F.Cu") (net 5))
 (segment (start 71.5 68.5194) (end 71.5 62.4) (width 0.6) (layer "F.Cu") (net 5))
 (segment (start 70.77 61.67) (end 66.38 61.67) (width 0.6) (layer "F.Cu") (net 5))
 (segment (start 72.0456 69.065) (end 71.5 68.5194) (width 0.6) (layer "F.Cu") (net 5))
 (segment (start 71.5 62.4) (end 70.77 61.67) (width 0.6) (layer "F.Cu") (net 5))
 (segment (start 71.135 55.965) (end 70.5 56.6) (width 0.6) (layer "F.Cu") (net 7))
 (segment (start 70.49 56.59) (end 66.38 56.59) (width 0.6) (layer "F.Cu") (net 7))
 (segment (start 73.67585 55.965) (end 71.135 55.965) (width 0.6) (layer "F.Cu") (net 7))
 (segment (start 70.5 56.6) (end 70.49 56.59) (width 0.6) (layer "F.Cu") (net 7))
 (segment (start 71.095 58.505) (end 73.67585 58.505) (width 0.6) (layer "F.Cu") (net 6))
 (segment (start 66.38 59.13) (end 70.47 59.13) (width 0.6) (layer "F.Cu") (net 6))
 (segment (start 70.47 59.13) (end 71.095 58.505) (width 0.6) (layer "F.Cu") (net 6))
 (segment (start 72.105 71.605) (end 70.2 69.7) (width 0.6) (layer "F.Cu") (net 4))
 (segment (start 70.2 69.7) (end 70.2 65.6) (width 0.6) (layer "F.Cu") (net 4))
 (segment (start 70.2 65.6) (end 68.81 64.21) (width 0.6) (layer "F.Cu") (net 4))
 (segment (start 73.37585 71.605) (end 72.105 71.605) (width 0.6) (layer "F.Cu") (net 4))
 (segment (start 68.81 64.21) (end 66.38 64.21) (width 0.6) (layer "F.Cu") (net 4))
 (segment (start 79.905 58.505) (end 79.12415 58.505) (width 0.4) (layer "F.Cu") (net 2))
 (segment (start 79.4 61.5) (end 80.2 60.7) (width 0.4) (layer "F.Cu") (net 2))
 (segment (start 84.476506 64.07) (end 81.97 64.07) (width 0.4) (layer "F.Cu") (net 2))
 (segment (start 77.6478 61.5) (end 79.4 61.5) (width 0.4) (layer "F.Cu") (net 2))
 (segment (start 80.2 58.8) (end 79.905 58.505) (width 0.4) (layer "F.Cu") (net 2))
 (segment (start 80.2 60.7) (end 80.2 58.8) (width 0.4) (layer "F.Cu") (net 2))
 (segment (start 81.97 64.07) (end 79.4 61.5) (width 0.4) (layer "F.Cu") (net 2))
 (segment (start 79.905 71.605) (end 80.2 71.9) (width 0.4) (layer "F.Cu") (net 8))
 (segment (start 77.7478 74.6) (end 78.7 74.6) (width 0.4) (layer "F.Cu") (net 8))
 (segment (start 78.7 74.6) (end 80.2 73.1) (width 0.4) (layer "F.Cu") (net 8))
 (segment (start 78.82415 71.605) (end 79.905 71.605) (width 0.4) (layer "F.Cu") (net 8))
 (segment (start 80.2 71.9) (end 80.2 73.1) (width 0.4) (layer "F.Cu") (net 8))
 (segment (start 84.476506 58.99) (end 84.39 58.99) (width 0.4) (layer "F.Cu") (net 10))
 (segment (start 82.7 58.3) (end 83.786506 58.3) (width 0.4) (layer "F.Cu") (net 10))
 (segment (start 84.39 58.99) (end 83.8 58.4) (width 0.4) (layer "F.Cu") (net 10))
 (segment (start 83.786506 58.3) (end 84.476506 58.99) (width 0.4) (layer "F.Cu") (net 10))
 (segment (start 80.365 55.965) (end 82.7 58.3) (width 0.4) (layer "F.Cu") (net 10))
 (segment (start 79.12415 55.965) (end 80.365 55.965) (width 0.4) (layer "F.Cu") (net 10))
 (segment (start 78.82415 67.795) (end 80.305 67.795) (width 0.4) (layer "F.Cu") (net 14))
 (segment (start 84.476506 66.61) (end 81.51 66.61) (width 0.4) (layer "F.Cu") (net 14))
 (segment (start 80.305 67.795) (end 81.5 66.6) (width 0.4) (layer "F.Cu") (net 14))
 (segment (start 81.51 66.61) (end 81.5 66.6) (width 0.4) (layer "F.Cu") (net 14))
 (segment (start 84.391506 69.065) (end 84.476506 69.15) (width 0.4) (layer "F.Cu") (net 13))
 (segment (start 78.82415 69.065) (end 84.391506 69.065) (width 0.4) (layer "F.Cu") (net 13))
 (segment (start 82.03 61.53) (end 84.476506 61.53) (width 0.4) (layer "F.Cu") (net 9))
 (segment (start 82 58.9806) (end 82 61.5) (width 0.4) (layer "F.Cu") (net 9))
 (segment (start 80.2544 57.235) (end 82 58.9806) (width 0.4) (layer "F.Cu") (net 9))
 (segment (start 79.12415 57.235) (end 80.2544 57.235) (width 0.4) (layer "F.Cu") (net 9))
 (segment (start 82 61.5) (end 82.03 61.53) (width 0.4) (layer "F.Cu") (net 9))
 (segment (start 84.476506 56.45) (end 82.85 56.45) (width 0.4) (layer "F.Cu") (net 11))
 (segment (start 81.095 54.695) (end 79.12415 54.695) (width 0.4) (layer "F.Cu") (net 11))
 (segment (start 82.85 56.45) (end 81.095 54.695) (width 0.4) (layer "F.Cu") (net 11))
 (segment (start 82.29 71.69) (end 84.476506 71.69) (width 0.4) (layer "F.Cu") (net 12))
 (segment (start 78.82415 70.335) (end 80.935 70.335) (width 0.4) (layer "F.Cu") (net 12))
 (segment (start 80.935 70.335) (end 82.29 71.69) (width 0.4) (layer "F.Cu") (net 12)))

